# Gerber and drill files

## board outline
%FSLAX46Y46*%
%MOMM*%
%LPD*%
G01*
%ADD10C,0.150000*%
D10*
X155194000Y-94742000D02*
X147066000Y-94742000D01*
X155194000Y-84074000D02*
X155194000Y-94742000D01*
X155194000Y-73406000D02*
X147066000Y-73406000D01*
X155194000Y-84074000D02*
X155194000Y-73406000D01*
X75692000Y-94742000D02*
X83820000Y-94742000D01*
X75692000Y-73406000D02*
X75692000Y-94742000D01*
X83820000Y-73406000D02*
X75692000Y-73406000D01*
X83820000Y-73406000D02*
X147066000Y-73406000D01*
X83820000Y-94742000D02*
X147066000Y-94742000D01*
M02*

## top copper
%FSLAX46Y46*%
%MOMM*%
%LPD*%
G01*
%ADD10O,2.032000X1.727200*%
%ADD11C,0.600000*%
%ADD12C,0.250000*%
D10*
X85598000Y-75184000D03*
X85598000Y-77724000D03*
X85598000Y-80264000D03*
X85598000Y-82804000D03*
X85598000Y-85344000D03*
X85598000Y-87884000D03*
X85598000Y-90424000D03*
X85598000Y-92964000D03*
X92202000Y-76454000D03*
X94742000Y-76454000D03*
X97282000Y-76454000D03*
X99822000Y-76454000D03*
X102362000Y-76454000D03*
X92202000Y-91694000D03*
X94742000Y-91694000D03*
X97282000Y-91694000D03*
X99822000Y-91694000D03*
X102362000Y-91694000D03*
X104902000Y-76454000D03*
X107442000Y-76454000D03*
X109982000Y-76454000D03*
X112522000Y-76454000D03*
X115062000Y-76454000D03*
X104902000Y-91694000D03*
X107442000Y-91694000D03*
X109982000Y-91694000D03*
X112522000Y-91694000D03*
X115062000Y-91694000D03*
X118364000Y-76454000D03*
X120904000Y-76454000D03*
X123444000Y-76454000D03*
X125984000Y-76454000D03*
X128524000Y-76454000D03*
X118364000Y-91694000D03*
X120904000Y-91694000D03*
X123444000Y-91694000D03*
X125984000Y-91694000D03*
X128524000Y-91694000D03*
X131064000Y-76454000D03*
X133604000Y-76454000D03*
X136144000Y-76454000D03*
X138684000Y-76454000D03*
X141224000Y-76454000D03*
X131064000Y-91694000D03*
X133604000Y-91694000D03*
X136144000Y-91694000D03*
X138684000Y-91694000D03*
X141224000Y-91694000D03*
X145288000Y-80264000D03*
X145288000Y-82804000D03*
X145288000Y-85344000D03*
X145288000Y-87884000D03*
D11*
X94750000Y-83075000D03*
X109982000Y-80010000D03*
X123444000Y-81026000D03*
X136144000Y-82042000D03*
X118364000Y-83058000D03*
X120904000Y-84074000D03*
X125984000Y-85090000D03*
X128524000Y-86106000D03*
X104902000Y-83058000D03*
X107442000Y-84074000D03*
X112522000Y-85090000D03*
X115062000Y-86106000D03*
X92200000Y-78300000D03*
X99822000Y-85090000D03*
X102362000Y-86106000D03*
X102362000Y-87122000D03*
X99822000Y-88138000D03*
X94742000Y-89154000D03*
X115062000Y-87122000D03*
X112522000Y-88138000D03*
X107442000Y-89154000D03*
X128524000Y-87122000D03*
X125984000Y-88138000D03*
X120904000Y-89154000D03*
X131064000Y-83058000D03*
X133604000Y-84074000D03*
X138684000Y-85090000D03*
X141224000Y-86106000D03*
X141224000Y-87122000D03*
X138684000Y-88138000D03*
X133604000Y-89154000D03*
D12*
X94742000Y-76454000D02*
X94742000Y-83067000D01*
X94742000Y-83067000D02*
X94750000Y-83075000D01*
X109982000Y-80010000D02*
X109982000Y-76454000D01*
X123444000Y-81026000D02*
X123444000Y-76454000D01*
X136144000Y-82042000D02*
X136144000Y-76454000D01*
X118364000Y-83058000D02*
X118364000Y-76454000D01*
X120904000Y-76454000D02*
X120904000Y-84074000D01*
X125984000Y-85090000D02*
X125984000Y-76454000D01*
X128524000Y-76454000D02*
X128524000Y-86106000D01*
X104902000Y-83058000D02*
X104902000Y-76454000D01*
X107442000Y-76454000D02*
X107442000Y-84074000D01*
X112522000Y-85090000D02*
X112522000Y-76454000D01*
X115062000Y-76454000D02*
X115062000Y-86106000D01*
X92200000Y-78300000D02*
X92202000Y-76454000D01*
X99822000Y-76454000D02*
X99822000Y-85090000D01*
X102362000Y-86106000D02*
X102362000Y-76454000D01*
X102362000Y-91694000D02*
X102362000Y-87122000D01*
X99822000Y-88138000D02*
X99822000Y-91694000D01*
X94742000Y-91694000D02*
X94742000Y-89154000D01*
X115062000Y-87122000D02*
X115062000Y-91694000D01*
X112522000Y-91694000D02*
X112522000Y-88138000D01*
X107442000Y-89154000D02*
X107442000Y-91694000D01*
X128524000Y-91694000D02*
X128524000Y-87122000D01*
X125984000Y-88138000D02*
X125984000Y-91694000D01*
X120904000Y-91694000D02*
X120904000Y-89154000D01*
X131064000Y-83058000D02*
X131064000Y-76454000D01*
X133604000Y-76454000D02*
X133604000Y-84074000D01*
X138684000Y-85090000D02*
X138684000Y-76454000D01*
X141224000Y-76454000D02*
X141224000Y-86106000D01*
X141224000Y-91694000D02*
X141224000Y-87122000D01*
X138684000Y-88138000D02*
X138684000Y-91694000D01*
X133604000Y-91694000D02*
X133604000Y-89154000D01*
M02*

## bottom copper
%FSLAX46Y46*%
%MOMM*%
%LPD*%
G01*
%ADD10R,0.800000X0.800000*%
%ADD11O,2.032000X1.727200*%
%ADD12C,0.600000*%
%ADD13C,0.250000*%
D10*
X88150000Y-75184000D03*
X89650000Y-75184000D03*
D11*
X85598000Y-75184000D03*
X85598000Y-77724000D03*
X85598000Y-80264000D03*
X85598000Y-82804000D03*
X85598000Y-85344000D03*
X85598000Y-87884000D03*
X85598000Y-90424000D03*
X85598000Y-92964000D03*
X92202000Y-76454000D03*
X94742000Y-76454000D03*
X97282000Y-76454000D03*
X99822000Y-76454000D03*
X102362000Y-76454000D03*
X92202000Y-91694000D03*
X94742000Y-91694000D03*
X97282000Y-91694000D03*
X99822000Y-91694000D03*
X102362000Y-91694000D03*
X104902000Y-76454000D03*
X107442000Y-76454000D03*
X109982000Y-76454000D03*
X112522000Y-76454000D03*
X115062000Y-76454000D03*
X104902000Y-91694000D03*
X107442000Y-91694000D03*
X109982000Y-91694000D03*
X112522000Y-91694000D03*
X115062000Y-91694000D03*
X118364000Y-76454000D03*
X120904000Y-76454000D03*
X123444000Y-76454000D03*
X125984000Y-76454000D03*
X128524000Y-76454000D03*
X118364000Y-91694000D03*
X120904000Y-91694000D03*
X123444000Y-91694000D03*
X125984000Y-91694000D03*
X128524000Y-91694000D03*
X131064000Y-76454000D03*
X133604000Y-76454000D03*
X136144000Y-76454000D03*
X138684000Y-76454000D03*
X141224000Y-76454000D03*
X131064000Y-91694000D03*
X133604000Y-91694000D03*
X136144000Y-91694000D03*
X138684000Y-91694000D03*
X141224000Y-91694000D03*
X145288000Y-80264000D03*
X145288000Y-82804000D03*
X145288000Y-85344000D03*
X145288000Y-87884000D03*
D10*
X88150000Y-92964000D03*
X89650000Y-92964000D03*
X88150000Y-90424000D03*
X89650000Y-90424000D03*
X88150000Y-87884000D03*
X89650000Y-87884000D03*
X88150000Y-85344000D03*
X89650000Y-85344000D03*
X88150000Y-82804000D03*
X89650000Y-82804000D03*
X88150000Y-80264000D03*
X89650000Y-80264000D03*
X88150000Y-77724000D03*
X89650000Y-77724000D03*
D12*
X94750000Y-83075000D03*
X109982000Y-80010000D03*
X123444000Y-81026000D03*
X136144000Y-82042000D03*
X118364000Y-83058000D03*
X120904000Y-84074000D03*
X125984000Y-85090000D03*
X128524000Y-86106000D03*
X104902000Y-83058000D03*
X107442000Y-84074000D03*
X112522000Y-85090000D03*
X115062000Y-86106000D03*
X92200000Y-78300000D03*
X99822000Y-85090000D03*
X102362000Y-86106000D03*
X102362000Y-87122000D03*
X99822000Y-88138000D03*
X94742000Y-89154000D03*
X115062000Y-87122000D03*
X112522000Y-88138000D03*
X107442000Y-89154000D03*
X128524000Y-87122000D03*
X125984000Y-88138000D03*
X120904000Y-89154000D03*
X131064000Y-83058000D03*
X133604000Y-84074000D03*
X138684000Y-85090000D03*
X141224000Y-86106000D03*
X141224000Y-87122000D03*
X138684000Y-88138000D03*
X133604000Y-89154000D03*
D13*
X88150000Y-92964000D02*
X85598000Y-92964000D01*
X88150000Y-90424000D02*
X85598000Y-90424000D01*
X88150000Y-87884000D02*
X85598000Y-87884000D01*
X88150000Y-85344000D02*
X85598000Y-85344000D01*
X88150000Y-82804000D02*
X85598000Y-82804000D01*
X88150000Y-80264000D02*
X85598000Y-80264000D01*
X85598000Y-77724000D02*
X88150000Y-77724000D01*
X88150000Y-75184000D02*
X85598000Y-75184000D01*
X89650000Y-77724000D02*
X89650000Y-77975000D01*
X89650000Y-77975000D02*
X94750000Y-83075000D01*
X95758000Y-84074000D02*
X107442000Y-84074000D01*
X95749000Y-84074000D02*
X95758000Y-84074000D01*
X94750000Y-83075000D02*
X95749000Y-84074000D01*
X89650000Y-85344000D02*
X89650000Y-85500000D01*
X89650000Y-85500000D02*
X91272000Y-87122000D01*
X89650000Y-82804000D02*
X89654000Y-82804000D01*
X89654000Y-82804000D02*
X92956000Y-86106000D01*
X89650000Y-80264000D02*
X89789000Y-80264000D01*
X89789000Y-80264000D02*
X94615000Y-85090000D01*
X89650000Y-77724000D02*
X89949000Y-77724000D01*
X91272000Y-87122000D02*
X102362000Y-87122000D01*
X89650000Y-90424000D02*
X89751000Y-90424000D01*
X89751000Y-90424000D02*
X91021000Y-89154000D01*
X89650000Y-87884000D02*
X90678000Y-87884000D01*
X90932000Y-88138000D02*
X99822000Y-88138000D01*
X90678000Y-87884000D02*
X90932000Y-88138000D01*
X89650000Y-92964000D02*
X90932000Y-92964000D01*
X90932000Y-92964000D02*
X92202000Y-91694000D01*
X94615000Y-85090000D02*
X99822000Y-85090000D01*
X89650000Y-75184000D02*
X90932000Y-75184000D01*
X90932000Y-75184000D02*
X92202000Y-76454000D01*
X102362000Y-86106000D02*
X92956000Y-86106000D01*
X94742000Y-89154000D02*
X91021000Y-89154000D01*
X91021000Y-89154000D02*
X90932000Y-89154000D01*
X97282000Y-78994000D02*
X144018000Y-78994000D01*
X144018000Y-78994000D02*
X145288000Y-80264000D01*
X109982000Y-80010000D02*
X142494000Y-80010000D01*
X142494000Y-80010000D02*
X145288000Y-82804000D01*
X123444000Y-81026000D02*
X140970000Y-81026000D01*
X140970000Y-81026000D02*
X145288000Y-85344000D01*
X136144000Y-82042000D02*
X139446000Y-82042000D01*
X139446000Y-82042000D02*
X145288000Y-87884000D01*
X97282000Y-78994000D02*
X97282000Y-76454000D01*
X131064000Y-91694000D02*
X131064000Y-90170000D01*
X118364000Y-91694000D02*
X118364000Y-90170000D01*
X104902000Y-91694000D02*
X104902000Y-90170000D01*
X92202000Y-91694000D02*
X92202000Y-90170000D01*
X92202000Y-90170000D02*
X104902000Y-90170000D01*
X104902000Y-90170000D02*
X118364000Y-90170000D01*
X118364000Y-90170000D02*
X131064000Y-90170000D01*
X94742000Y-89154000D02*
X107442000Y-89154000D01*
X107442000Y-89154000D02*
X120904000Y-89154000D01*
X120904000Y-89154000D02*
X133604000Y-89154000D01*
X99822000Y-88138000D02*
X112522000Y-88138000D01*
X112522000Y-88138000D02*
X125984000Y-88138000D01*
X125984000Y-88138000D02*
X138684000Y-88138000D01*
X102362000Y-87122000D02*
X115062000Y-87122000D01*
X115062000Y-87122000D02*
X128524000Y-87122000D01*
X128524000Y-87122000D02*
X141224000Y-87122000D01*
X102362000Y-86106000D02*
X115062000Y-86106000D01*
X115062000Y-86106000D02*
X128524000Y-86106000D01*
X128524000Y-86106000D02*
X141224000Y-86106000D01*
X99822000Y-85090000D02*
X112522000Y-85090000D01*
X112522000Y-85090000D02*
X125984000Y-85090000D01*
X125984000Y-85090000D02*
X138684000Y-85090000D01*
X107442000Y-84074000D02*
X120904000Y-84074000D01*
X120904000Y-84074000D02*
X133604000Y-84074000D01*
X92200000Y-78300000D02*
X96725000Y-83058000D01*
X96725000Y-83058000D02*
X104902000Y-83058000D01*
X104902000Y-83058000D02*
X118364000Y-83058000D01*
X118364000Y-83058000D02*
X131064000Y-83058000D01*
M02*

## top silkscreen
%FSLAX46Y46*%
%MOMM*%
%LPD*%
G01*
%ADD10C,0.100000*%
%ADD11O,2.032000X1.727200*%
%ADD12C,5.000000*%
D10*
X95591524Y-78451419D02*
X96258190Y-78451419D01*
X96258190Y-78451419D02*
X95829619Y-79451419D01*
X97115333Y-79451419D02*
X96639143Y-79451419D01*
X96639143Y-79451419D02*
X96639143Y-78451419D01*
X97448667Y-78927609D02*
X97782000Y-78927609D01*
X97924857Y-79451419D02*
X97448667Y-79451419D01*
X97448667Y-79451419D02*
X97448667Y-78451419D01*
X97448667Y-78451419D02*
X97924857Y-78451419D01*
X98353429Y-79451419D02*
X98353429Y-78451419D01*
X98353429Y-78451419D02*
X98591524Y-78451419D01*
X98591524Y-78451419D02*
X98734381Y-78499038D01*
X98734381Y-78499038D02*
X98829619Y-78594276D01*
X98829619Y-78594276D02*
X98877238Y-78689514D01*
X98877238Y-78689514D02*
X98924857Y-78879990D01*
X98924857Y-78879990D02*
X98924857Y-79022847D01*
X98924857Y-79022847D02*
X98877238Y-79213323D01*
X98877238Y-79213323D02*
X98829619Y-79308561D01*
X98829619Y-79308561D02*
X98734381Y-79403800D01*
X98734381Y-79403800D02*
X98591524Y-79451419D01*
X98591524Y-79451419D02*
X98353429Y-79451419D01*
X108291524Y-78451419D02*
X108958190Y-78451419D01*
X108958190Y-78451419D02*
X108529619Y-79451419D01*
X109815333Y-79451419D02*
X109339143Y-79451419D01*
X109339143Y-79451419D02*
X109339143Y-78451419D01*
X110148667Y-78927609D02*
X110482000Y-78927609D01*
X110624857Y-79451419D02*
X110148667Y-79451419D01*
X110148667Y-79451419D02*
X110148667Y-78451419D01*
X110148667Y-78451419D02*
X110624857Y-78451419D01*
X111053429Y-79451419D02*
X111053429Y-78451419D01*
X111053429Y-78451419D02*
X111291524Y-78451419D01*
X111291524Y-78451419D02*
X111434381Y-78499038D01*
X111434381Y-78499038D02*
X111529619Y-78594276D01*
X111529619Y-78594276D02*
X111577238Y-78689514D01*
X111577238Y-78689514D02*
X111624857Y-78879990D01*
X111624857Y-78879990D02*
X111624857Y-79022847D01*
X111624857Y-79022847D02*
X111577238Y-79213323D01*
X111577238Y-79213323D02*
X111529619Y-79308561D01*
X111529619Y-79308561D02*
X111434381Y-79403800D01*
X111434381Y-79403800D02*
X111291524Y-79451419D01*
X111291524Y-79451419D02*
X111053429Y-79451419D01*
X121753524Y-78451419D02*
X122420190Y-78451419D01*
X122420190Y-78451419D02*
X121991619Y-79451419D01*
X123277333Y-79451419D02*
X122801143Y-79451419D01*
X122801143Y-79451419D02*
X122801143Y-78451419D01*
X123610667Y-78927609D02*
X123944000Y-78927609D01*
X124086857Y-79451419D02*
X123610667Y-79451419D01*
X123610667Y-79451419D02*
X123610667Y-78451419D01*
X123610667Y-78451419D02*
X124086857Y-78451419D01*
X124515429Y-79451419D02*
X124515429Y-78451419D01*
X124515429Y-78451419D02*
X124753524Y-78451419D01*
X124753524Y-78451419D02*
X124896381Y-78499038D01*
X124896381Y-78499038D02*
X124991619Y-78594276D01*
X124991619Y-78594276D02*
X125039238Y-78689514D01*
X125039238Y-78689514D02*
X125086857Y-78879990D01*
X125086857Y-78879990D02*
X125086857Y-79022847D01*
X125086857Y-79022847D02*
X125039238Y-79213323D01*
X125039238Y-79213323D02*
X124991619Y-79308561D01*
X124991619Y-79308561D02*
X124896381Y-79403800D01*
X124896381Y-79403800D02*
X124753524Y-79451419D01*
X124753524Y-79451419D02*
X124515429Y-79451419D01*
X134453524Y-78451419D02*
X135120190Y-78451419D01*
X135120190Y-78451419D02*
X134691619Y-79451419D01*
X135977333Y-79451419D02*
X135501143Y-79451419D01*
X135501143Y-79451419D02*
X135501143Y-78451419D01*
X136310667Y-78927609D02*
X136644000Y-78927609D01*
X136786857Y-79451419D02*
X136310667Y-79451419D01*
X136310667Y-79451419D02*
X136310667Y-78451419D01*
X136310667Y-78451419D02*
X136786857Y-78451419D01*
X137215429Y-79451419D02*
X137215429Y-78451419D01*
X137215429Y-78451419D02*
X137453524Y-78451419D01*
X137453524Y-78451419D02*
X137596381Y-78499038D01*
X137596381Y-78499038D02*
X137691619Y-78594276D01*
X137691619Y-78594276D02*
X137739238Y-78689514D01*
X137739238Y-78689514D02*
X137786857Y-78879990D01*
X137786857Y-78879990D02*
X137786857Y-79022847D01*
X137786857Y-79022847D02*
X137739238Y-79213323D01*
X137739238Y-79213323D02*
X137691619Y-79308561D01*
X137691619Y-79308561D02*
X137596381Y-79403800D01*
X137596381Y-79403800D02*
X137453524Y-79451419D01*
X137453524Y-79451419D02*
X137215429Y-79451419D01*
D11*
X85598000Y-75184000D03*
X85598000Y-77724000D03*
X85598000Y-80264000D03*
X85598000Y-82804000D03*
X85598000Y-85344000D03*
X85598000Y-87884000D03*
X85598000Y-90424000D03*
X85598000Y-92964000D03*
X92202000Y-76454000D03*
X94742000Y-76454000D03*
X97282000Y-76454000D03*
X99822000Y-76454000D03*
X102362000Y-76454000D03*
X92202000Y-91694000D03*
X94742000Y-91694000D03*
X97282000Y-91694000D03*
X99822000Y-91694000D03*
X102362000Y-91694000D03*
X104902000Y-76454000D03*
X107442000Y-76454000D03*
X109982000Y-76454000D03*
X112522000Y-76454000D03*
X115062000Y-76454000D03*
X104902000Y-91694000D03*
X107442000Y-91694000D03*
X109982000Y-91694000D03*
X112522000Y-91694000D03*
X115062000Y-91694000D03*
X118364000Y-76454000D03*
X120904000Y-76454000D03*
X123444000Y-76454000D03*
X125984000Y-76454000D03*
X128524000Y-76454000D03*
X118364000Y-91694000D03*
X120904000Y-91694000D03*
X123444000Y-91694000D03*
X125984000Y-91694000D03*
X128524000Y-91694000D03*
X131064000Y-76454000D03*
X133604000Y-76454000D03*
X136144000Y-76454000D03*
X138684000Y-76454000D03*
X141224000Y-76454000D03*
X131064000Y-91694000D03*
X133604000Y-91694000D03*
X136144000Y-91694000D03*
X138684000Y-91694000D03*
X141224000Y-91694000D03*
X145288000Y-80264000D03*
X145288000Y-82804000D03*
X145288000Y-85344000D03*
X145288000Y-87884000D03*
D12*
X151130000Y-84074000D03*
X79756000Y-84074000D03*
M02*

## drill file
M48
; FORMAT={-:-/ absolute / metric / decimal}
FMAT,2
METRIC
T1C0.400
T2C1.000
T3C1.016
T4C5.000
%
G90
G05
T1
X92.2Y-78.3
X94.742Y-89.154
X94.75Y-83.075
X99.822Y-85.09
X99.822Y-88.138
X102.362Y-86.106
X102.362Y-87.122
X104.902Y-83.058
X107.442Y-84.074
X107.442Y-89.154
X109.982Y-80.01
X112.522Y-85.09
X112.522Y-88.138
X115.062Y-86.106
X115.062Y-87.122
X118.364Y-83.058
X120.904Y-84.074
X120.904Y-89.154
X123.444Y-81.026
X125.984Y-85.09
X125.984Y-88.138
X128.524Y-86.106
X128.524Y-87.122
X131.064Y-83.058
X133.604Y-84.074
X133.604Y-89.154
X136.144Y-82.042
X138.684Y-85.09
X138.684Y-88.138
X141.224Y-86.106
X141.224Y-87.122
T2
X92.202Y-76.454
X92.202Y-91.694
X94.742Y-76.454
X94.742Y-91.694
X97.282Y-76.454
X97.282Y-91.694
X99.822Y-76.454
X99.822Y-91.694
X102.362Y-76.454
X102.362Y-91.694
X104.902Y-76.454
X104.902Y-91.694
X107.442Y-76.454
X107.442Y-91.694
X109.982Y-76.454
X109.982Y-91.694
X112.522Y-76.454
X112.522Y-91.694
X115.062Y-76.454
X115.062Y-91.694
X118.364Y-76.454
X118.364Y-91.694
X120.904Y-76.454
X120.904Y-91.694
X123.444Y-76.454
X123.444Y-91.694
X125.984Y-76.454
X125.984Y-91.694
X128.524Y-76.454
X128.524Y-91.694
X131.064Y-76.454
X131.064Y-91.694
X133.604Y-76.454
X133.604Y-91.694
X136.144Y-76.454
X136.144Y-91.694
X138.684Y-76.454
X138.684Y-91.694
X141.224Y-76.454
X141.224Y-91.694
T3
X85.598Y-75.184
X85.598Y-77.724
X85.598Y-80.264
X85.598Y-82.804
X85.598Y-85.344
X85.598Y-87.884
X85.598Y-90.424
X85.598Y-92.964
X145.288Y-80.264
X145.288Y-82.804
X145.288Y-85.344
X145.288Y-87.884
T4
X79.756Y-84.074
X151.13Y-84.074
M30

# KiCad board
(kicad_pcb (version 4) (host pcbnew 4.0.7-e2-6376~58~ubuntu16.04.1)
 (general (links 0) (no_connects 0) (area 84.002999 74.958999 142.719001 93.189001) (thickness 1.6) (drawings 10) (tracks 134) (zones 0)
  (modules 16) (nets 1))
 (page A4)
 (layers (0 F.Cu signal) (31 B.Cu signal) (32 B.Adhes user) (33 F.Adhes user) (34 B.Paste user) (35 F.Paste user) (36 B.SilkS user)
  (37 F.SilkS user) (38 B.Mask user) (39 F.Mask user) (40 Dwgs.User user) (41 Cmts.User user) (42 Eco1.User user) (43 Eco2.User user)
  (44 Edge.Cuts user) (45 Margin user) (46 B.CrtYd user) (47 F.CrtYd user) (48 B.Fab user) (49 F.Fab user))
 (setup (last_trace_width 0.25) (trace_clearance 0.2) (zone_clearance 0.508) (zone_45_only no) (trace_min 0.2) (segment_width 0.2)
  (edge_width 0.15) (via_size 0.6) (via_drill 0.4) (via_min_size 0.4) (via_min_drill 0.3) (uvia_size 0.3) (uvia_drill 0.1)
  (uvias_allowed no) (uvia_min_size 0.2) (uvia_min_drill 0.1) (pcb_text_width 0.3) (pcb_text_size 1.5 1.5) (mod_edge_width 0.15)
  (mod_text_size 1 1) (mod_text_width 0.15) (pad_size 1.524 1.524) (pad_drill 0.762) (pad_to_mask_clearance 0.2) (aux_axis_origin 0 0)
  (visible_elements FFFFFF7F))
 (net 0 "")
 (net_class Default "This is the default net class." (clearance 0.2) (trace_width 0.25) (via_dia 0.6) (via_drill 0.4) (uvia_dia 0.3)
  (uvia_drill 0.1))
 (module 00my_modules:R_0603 (layer B.Cu) (at 88.9 75.184)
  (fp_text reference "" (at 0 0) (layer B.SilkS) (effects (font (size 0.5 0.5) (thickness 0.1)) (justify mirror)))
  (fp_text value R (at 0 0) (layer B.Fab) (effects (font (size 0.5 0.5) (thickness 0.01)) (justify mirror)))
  (pad 1 smd rect (at -0.75 0) (size 0.8 0.8) (layers B.Cu B.Paste B.Mask))
  (pad 2 smd rect (at 0.75 0) (size 0.8 0.8) (layers B.Cu B.Paste B.Mask)))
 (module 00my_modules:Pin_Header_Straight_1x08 (layer F.Cu) (at 85.598 75.184)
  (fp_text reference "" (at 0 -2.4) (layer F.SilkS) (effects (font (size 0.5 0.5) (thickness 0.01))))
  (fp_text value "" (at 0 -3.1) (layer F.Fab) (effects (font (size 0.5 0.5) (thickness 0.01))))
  (pad 1 thru_hole oval (at 0 0) (size 2.032 1.7272) (drill 1.016) (layers *.Cu *.Mask F.SilkS))
  (pad 2 thru_hole oval (at 0 2.54) (size 2.032 1.7272) (drill 1.016) (layers *.Cu *.Mask F.SilkS))
  (pad 3 thru_hole oval (at 0 5.08) (size 2.032 1.7272) (drill 1.016) (layers *.Cu *.Mask F.SilkS))
  (pad 4 thru_hole oval (at 0 7.62) (size 2.032 1.7272) (drill 1.016) (layers *.Cu *.Mask F.SilkS))
  (pad 5 thru_hole oval (at 0 10.16) (size 2.032 1.7272) (drill 1.016) (layers *.Cu *.Mask F.SilkS))
  (pad 6 thru_hole oval (at 0 12.7) (size 2.032 1.7272) (drill 1.016) (layers *.Cu *.Mask F.SilkS))
  (pad 7 thru_hole oval (at 0 15.24) (size 2.032 1.7272) (drill 1.016) (layers *.Cu *.Mask F.SilkS))
  (pad 8 thru_hole oval (at 0 17.78) (size 2.032 1.7272) (drill 1.016) (layers *.Cu *.Mask F.SilkS)))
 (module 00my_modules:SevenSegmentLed (layer F.Cu) (at 92.202 76.454)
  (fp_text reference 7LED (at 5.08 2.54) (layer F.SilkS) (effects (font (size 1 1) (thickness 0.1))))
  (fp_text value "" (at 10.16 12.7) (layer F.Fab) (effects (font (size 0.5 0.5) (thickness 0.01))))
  (pad 10 thru_hole oval (at 0 0) (size 2.032 1.7272) (drill 1) (layers *.Cu *.Mask F.SilkS))
  (pad 9 thru_hole oval (at 2.54 0) (size 2.032 1.7272) (drill 1) (layers *.Cu *.Mask F.SilkS))
  (pad 8 thru_hole oval (at 5.08 0) (size 2.032 1.7272) (drill 1) (layers *.Cu *.Mask F.SilkS))
  (pad 7 thru_hole oval (at 7.62 0) (size 2.032 1.7272) (drill 1) (layers *.Cu *.Mask F.SilkS))
  (pad 6 thru_hole oval (at 10.16 0) (size 2.032 1.7272) (drill 1) (layers *.Cu *.Mask F.SilkS))
  (pad 1 thru_hole oval (at 0 15.24) (size 2.032 1.7272) (drill 1) (layers *.Cu *.Mask F.SilkS))
  (pad 2 thru_hole oval (at 2.54 15.24) (size 2.032 1.7272) (drill 1) (layers *.Cu *.Mask F.SilkS))
  (pad 3 thru_hole oval (at 5.08 15.24) (size 2.032 1.7272) (drill 1) (layers *.Cu *.Mask F.SilkS))
  (pad 4 thru_hole oval (at 7.62 15.24) (size 2.032 1.7272) (drill 1) (layers *.Cu *.Mask F.SilkS))
  (pad 5 thru_hole oval (at 10.16 15.24) (size 2.032 1.7272) (drill 1) (layers *.Cu *.Mask F.SilkS)))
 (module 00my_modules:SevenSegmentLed (layer F.Cu) (at 104.902 76.454)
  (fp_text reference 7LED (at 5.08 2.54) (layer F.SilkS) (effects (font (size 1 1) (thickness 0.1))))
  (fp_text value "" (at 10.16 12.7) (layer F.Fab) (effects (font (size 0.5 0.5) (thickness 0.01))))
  (pad 10 thru_hole oval (at 0 0) (size 2.032 1.7272) (drill 1) (layers *.Cu *.Mask F.SilkS))
  (pad 9 thru_hole oval (at 2.54 0) (size 2.032 1.7272) (drill 1) (layers *.Cu *.Mask F.SilkS))
  (pad 8 thru_hole oval (at 5.08 0) (size 2.032 1.7272) (drill 1) (layers *.Cu *.Mask F.SilkS))
  (pad 7 thru_hole oval (at 7.62 0) (size 2.032 1.7272) (drill 1) (layers *.Cu *.Mask F.SilkS))
  (pad 6 thru_hole oval (at 10.16 0) (size 2.032 1.7272) (drill 1) (layers *.Cu *.Mask F.SilkS))
  (pad 1 thru_hole oval (at 0 15.24) (size 2.032 1.7272) (drill 1) (layers *.Cu *.Mask F.SilkS))
  (pad 2 thru_hole oval (at 2.54 15.24) (size 2.032 1.7272) (drill 1) (layers *.Cu *.Mask F.SilkS))
  (pad 3 thru_hole oval (at 5.08 15.24) (size 2.032 1.7272) (drill 1) (layers *.Cu *.Mask F.SilkS))
  (pad 4 thru_hole oval (at 7.62 15.24) (size 2.032 1.7272) (drill 1) (layers *.Cu *.Mask F.SilkS))
  (pad 5 thru_hole oval (at 10.16 15.24) (size 2.032 1.7272) (drill 1) (layers *.Cu *.Mask F.SilkS)))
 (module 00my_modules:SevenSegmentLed (layer F.Cu) (at 118.364 76.454)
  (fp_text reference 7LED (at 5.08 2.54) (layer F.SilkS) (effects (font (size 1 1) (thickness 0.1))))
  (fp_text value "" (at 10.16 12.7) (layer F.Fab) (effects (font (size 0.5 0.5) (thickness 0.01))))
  (pad 10 thru_hole oval (at 0 0) (size 2.032 1.7272) (drill 1) (layers *.Cu *.Mask F.SilkS))
  (pad 9 thru_hole oval (at 2.54 0) (size 2.032 1.7272) (drill 1) (layers *.Cu *.Mask F.SilkS))
  (pad 8 thru_hole oval (at 5.08 0) (size 2.032 1.7272) (drill 1) (layers *.Cu *.Mask F.SilkS))
  (pad 7 thru_hole oval (at 7.62 0) (size 2.032 1.7272) (drill 1) (layers *.Cu *.Mask F.SilkS))
  (pad 6 thru_hole oval (at 10.16 0) (size 2.032 1.7272) (drill 1) (layers *.Cu *.Mask F.SilkS))
  (pad 1 thru_hole oval (at 0 15.24) (size 2.032 1.7272) (drill 1) (layers *.Cu *.Mask F.SilkS))
  (pad 2 thru_hole oval (at 2.54 15.24) (size 2.032 1.7272) (drill 1) (layers *.Cu *.Mask F.SilkS))
  (pad 3 thru_hole oval (at 5.08 15.24) (size 2.032 1.7272) (drill 1) (layers *.Cu *.Mask F.SilkS))
  (pad 4 thru_hole oval (at 7.62 15.24) (size 2.032 1.7272) (drill 1) (layers *.Cu *.Mask F.SilkS))
  (pad 5 thru_hole oval (at 10.16 15.24) (size 2.032 1.7272) (drill 1) (layers *.Cu *.Mask F.SilkS)))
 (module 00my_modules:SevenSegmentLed (layer F.Cu) (at 131.064 76.454)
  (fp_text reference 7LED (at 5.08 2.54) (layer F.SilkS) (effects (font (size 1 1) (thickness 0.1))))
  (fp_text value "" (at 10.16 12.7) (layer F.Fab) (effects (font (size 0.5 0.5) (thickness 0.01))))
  (pad 10 thru_hole oval (at 0 0) (size 2.032 1.7272) (drill 1) (layers *.Cu *.Mask F.SilkS))
  (pad 9 thru_hole oval (at 2.54 0) (size 2.032 1.7272) (drill 1) (layers *.Cu *.Mask F.SilkS))
  (pad 8 thru_hole oval (at 5.08 0) (size 2.032 1.7272) (drill 1) (layers *.Cu *.Mask F.SilkS))
  (pad 7 thru_hole oval (at 7.62 0) (size 2.032 1.7272) (drill 1) (layers *.Cu *.Mask F.SilkS))
  (pad 6 thru_hole oval (at 10.16 0) (size 2.032 1.7272) (drill 1) (layers *.Cu *.Mask F.SilkS))
  (pad 1 thru_hole oval (at 0 15.24) (size 2.032 1.7272) (drill 1) (layers *.Cu *.Mask F.SilkS))
  (pad 2 thru_hole oval (at 2.54 15.24) (size 2.032 1.7272) (drill 1) (layers *.Cu *.Mask F.SilkS))
  (pad 3 thru_hole oval (at 5.08 15.24) (size 2.032 1.7272) (drill 1) (layers *.Cu *.Mask F.SilkS))
  (pad 4 thru_hole oval (at 7.62 15.24) (size 2.032 1.7272) (drill 1) (layers *.Cu *.Mask F.SilkS))
  (pad 5 thru_hole oval (at 10.16 15.24) (size 2.032 1.7272) (drill 1) (layers *.Cu *.Mask F.SilkS)))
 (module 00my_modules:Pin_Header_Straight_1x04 (layer F.Cu) (at 145.288 80.264)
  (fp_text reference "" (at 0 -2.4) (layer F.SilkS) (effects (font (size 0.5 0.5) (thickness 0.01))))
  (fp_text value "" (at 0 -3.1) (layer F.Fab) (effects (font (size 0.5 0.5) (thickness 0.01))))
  (pad 1 thru_hole oval (at 0 0) (size 2.032 1.7272) (drill 1.016) (layers *.Cu *.Mask F.SilkS))
  (pad 2 thru_hole oval (at 0 2.54) (size 2.032 1.7272) (drill 1.016) (layers *.Cu *.Mask F.SilkS))
  (pad 3 thru_hole oval (at 0 5.08) (size 2.032 1.7272) (drill 1.016) (layers *.Cu *.Mask F.SilkS))
  (pad 4 thru_hole oval (at 0 7.62) (size 2.032 1.7272) (drill 1.016) (layers *.Cu *.Mask F.SilkS)))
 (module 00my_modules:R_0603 (layer B.Cu) (at 88.9 92.964)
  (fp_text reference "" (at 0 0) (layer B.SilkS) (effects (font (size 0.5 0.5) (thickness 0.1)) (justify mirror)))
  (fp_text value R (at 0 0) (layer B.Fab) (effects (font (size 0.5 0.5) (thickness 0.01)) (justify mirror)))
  (pad 1 smd rect (at -0.75 0) (size 0.8 0.8) (layers B.Cu B.Paste B.Mask))
  (pad 2 smd rect (at 0.75 0) (size 0.8 0.8) (layers B.Cu B.Paste B.Mask)))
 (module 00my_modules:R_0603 (layer B.Cu) (at 88.9 90.424)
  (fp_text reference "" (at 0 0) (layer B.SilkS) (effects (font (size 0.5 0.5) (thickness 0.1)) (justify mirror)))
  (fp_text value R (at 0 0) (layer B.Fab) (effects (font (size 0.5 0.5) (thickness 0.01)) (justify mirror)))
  (pad 1 smd rect (at -0.75 0) (size 0.8 0.8) (layers B.Cu B.Paste B.Mask))
  (pad 2 smd rect (at 0.75 0) (size 0.8 0.8) (layers B.Cu B.Paste B.Mask)))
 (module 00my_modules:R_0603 (layer B.Cu) (at 88.9 87.884)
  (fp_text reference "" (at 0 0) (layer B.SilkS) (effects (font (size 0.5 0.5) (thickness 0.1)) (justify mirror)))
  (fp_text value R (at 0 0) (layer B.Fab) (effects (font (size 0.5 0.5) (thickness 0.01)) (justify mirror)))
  (pad 1 smd rect (at -0.75 0) (size 0.8 0.8) (layers B.Cu B.Paste B.Mask))
  (pad 2 smd rect (at 0.75 0) (size 0.8 0.8) (layers B.Cu B.Paste B.Mask)))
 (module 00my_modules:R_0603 (layer B.Cu) (at 88.9 85.344)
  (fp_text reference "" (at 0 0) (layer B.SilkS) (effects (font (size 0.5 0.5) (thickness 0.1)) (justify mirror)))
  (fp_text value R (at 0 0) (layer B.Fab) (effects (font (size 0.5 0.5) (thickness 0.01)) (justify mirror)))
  (pad 1 smd rect (at -0.75 0) (size 0.8 0.8) (layers B.Cu B.Paste B.Mask))
  (pad 2 smd rect (at 0.75 0) (size 0.8 0.8) (layers B.Cu B.Paste B.Mask)))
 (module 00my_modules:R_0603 (layer B.Cu) (at 88.9 82.804)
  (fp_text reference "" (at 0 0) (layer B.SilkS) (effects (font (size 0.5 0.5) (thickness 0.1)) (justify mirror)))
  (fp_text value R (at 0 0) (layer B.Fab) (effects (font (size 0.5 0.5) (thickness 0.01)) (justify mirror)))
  (pad 1 smd rect (at -0.75 0) (size 0.8 0.8) (layers B.Cu B.Paste B.Mask))
  (pad 2 smd rect (at 0.75 0) (size 0.8 0.8) (layers B.Cu B.Paste B.Mask)))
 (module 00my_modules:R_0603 (layer B.Cu) (at 88.9 80.264)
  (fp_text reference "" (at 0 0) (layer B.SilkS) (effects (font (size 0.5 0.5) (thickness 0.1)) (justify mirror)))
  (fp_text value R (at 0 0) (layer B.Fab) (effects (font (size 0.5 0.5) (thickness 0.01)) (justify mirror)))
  (pad 1 smd rect (at -0.75 0) (size 0.8 0.8) (layers B.Cu B.Paste B.Mask))
  (pad 2 smd rect (at 0.75 0) (size 0.8 0.8) (layers B.Cu B.Paste B.Mask)))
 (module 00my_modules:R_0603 (layer B.Cu) (at 88.9 77.724)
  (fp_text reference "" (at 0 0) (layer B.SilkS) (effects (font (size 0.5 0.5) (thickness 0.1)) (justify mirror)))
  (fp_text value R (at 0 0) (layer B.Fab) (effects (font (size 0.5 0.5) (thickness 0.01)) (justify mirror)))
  (pad 1 smd rect (at -0.75 0) (size 0.8 0.8) (layers B.Cu B.Paste B.Mask))
  (pad 2 smd rect (at 0.75 0) (size 0.8 0.8) (layers B.Cu B.Paste B.Mask)))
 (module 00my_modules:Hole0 (layer F.Cu) (at 151.13 84.074)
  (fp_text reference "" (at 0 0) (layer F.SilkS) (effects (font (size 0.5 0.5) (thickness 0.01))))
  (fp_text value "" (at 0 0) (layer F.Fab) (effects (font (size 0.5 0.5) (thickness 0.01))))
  (pad "" np_thru_hole circle (at 0 0) (size 5 5) (drill 5) (layers *.Cu *.Mask F.SilkS)))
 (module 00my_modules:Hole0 (layer F.Cu) (at 79.756 84.074)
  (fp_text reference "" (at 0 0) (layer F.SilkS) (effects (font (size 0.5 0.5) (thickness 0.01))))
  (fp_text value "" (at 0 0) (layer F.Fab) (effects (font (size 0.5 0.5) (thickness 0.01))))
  (pad "" np_thru_hole circle (at 0 0) (size 5 5) (drill 5) (layers *.Cu *.Mask F.SilkS)))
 (gr_line (start 155.194 94.742) (end 147.066 94.742) (angle 90) (layer Edge.Cuts) (width 0.15))
 (gr_line (start 155.194 84.074) (end 155.194 94.742) (angle 90) (layer Edge.Cuts) (width 0.15))
 (gr_line (start 155.194 73.406) (end 147.066 73.406) (angle 90) (layer Edge.Cuts) (width 0.15))
 (gr_line (start 155.194 84.074) (end 155.194 73.406) (angle 90) (layer Edge.Cuts) (width 0.15))
 (gr_line (start 75.692 94.742) (end 83.82 94.742) (angle 90) (layer Edge.Cuts) (width 0.15))
 (gr_line (start 75.692 73.406) (end 75.692 94.742) (angle 90) (layer Edge.Cuts) (width 0.15))
 (gr_line (start 83.82 73.406) (end 75.692 73.406) (angle 90) (layer Edge.Cuts) (width 0.15))
 (gr_line (start 83.82 73.406) (end 147.066 73.406) (angle 90) (layer Edge.Cuts) (width 0.15))
 (gr_line (start 83.82 94.742) (end 147.066 94.742) (angle 90) (layer Edge.Cuts) (width 0.15))
 (segment (start 88.15 92.964) (end 85.598 92.964) (width 0.25) (layer B.Cu) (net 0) (status C00000))
 (segment (start 88.15 90.424) (end 85.598 90.424) (width 0.25) (layer B.Cu) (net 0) (status C00000))
 (segment (start 88.15 87.884) (end 85.598 87.884) (width 0.25) (layer B.Cu) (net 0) (status C00000))
 (segment (start 88.15 85.344) (end 85.598 85.344) (width 0.25) (layer B.Cu) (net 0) (status C00000))
 (segment (start 88.15 82.804) (end 85.598 82.804) (width 0.25) (layer B.Cu) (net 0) (status C00000))
 (segment (start 88.15 80.264) (end 85.598 80.264) (width 0.25) (layer B.Cu) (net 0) (status C00000))
 (segment (start 85.598 77.724) (end 88.15 77.724) (width 0.25) (layer B.Cu) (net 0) (status C00000))
 (segment (start 88.15 75.184) (end 85.598 75.184) (width 0.25) (layer B.Cu) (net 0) (status C00000))
 (segment (start 89.65 77.724) (end 89.65 77.975) (width 0.25) (layer B.Cu) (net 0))
 (segment (start 89.65 77.975) (end 94.75 83.075) (width 0.25) (layer B.Cu) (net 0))
 (segment (start 94.742 76.454) (end 94.742 83.067) (width 0.25) (layer F.Cu) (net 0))
 (segment (start 95.758 84.074) (end 107.442 84.074) (width 0.25) (layer B.Cu) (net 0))
 (segment (start 95.749 84.074) (end 95.758 84.074) (width 0.25) (layer B.Cu) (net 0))
 (segment (start 94.75 83.075) (end 95.749 84.074) (width 0.25) (layer B.Cu) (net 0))
 (via (at 94.75 83.075) (size 0.6) (drill 0.4) (layers F.Cu B.Cu) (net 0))
 (segment (start 94.742 83.067) (end 94.75 83.075) (width 0.25) (layer F.Cu) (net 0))
 (segment (start 89.65 85.344) (end 89.65 85.5) (width 0.25) (layer B.Cu) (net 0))
 (segment (start 89.65 85.5) (end 91.272 87.122) (width 0.25) (layer B.Cu) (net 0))
 (segment (start 89.65 82.804) (end 89.654 82.804) (width 0.25) (layer B.Cu) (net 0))
 (segment (start 89.654 82.804) (end 92.956 86.106) (width 0.25) (layer B.Cu) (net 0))
 (segment (start 89.65 80.264) (end 89.789 80.264) (width 0.25) (layer B.Cu) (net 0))
 (segment (start 89.789 80.264) (end 94.615 85.09) (width 0.25) (layer B.Cu) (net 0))
 (segment (start 89.65 77.724) (end 89.949 77.724) (width 0.25) (layer B.Cu) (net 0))
 (segment (start 91.272 87.122) (end 102.362 87.122) (width 0.25) (layer B.Cu) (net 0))
 (segment (start 89.65 90.424) (end 89.751 90.424) (width 0.25) (layer B.Cu) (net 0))
 (segment (start 89.751 90.424) (end 91.021 89.154) (width 0.25) (layer B.Cu) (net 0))
 (segment (start 89.65 87.884) (end 90.678 87.884) (width 0.25) (layer B.Cu) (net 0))
 (segment (start 90.932 88.138) (end 99.822 88.138) (width 0.25) (layer B.Cu) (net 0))
 (segment (start 90.678 87.884) (end 90.932 88.138) (width 0.25) (layer B.Cu) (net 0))
 (segment (start 89.65 92.964) (end 90.932 92.964) (width 0.25) (layer B.Cu) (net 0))
 (segment (start 90.932 92.964) (end 92.202 91.694) (width 0.25) (layer B.Cu) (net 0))
 (segment (start 94.615 85.09) (end 99.822 85.09) (width 0.25) (layer B.Cu) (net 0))
 (segment (start 89.65 75.184) (end 90.932 75.184) (width 0.25) (layer B.Cu) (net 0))
 (segment (start 90.932 75.184) (end 92.202 76.454) (width 0.25) (layer B.Cu) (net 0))
 (segment (start 102.362 86.106) (end 92.956 86.106) (width 0.25) (layer B.Cu) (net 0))
 (segment (start 94.742 89.154) (end 91.021 89.154) (width 0.25) (layer B.Cu) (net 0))
 (segment (start 91.021 89.154) (end 90.932 89.154) (width 0.25) (layer B.Cu) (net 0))
 (segment (start 97.282 78.994) (end 144.018 78.994) (width 0.25) (layer B.Cu) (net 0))
 (segment (start 144.018 78.994) (end 145.288 80.264) (width 0.25) (layer B.Cu) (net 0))
 (segment (start 109.982 80.01) (end 142.494 80.01) (width 0.25) (layer B.Cu) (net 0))
 (segment (start 142.494 80.01) (end 145.288 82.804) (width 0.25) (layer B.Cu) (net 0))
 (segment (start 123.444 81.026) (end 140.97 81.026) (width 0.25) (layer B.Cu) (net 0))
 (segment (start 140.97 81.026) (end 145.288 85.344) (width 0.25) (layer B.Cu) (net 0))
 (segment (start 136.144 82.042) (end 139.446 82.042) (width 0.25) (layer B.Cu) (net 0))
 (segment (start 139.446 82.042) (end 145.288 87.884) (width 0.25) (layer B.Cu) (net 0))
 (segment (start 97.282 78.994) (end 97.282 76.454) (width 0.25) (layer B.Cu) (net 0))
 (via (at 109.982 80.01) (size 0.6) (drill 0.4) (layers F.Cu B.Cu) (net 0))
 (segment (start 109.982 80.01) (end 109.982 76.454) (width 0.25) (layer F.Cu) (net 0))
 (segment (start 123.444 81.026) (end 123.444 76.454) (width 0.25) (layer F.Cu) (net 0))
 (via (at 123.444 81.026) (size 0.6) (drill 0.4) (layers F.Cu B.Cu) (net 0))
 (via (at 136.144 82.042) (size 0.6) (drill 0.4) (layers F.Cu B.Cu) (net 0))
 (segment (start 136.144 82.042) (end 136.144 76.454) (width 0.25) (layer F.Cu) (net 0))
 (via (at 118.364 83.058) (size 0.6) (drill 0.4) (layers F.Cu B.Cu) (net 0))
 (segment (start 118.364 83.058) (end 118.364 76.454) (width 0.25) (layer F.Cu) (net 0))
 (segment (start 120.904 76.454) (end 120.904 84.074) (width 0.25) (layer F.Cu) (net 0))
 (via (at 120.904 84.074) (size 0.6) (drill 0.4) (layers F.Cu B.Cu) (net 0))
 (via (at 125.984 85.09) (size 0.6) (drill 0.4) (layers F.Cu B.Cu) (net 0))
 (segment (start 125.984 85.09) (end 125.984 76.454) (width 0.25) (layer F.Cu) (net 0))
 (segment (start 128.524 76.454) (end 128.524 86.106) (width 0.25) (layer F.Cu) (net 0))
 (via (at 128.524 86.106) (size 0.6) (drill 0.4) (layers F.Cu B.Cu) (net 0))
 (via (at 104.902 83.058) (size 0.6) (drill 0.4) (layers F.Cu B.Cu) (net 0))
 (segment (start 104.902 83.058) (end 104.902 76.454) (width 0.25) (layer F.Cu) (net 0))
 (segment (start 107.442 76.454) (end 107.442 84.074) (width 0.25) (layer F.Cu) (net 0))
 (via (at 107.442 84.074) (size 0.6) (drill 0.4) (layers F.Cu B.Cu) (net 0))
 (via (at 112.522 85.09) (size 0.6) (drill 0.4) (layers F.Cu B.Cu) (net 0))
 (segment (start 112.522 85.09) (end 112.522 76.454) (width 0.25) (layer F.Cu) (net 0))
 (segment (start 115.062 76.454) (end 115.062 86.106) (width 0.25) (layer F.Cu) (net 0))
 (via (at 115.062 86.106) (size 0.6) (drill 0.4) (layers F.Cu B.Cu) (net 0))
 (via (at 92.2 78.3) (size 0.6) (drill 0.4) (layers F.Cu B.Cu) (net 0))
 (segment (start 92.2 78.3) (end 92.202 76.454) (width 0.25) (layer F.Cu) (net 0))
 (segment (start 99.822 76.454) (end 99.822 85.09) (width 0.25) (layer F.Cu) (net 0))
 (via (at 99.822 85.09) (size 0.6) (drill 0.4) (layers F.Cu B.Cu) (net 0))
 (via (at 102.362 86.106) (size 0.6) (drill 0.4) (layers F.Cu B.Cu) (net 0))
 (segment (start 102.362 86.106) (end 102.362 76.454) (width 0.25) (layer F.Cu) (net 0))
 (segment (start 102.362 91.694) (end 102.362 87.122) (width 0.25) (layer F.Cu) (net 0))
 (via (at 102.362 87.122) (size 0.6) (drill 0.4) (layers F.Cu B.Cu) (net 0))
 (via (at 99.822 88.138) (size 0.6) (drill 0.4) (layers F.Cu B.Cu) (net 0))
 (segment (start 99.822 88.138) (end 99.822 91.694) (width 0.25) (layer F.Cu) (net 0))
 (segment (start 94.742 91.694) (end 94.742 89.154) (width 0.25) (layer F.Cu) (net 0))
 (via (at 94.742 89.154) (size 0.6) (drill 0.4) (layers F.Cu B.Cu) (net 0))
 (via (at 115.062 87.122) (size 0.6) (drill 0.4) (layers F.Cu B.Cu) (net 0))
 (segment (start 115.062 87.122) (end 115.062 91.694) (width 0.25) (layer F.Cu) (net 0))
 (segment (start 112.522 91.694) (end 112.522 88.138) (width 0.25) (layer F.Cu) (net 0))
 (via (at 112.522 88.138) (size 0.6) (drill 0.4) (layers F.Cu B.Cu) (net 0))
 (via (at 107.442 89.154) (size 0.6) (drill 0.4) (layers F.Cu B.Cu) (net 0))
 (segment (start 107.442 89.154) (end 107.442 91.694) (width 0.25) (layer F.Cu) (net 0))
 (segment (start 128.524 91.694) (end 128.524 87.122) (width 0.25) (layer F.Cu) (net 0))
 (via (at 128.524 87.122) (size 0.6) (drill 0.4) (layers F.Cu B.Cu) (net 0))
 (via (at 125.984 88.138) (size 0.6) (drill 0.4) (layers F.Cu B.Cu) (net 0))
 (segment (start 125.984 88.138) (end 125.984 91.694) (width 0.25) (layer F.Cu) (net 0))
 (segment (start 120.904 91.694) (end 120.904 89.154) (width 0.25) (layer F.Cu) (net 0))
 (via (at 120.904 89.154) (size 0.6) (drill 0.4) (layers F.Cu B.Cu) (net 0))
 (via (at 131.064 83.058) (size 0.6) (drill 0.4) (layers F.Cu B.Cu) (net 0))
 (segment (start 131.064 83.058) (end 131.064 76.454) (width 0.25) (layer F.Cu) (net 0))
 (segment (start 133.604 76.454) (end 133.604 84.074) (width 0.25) (layer F.Cu) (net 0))
 (via (at 133.604 84.074) (size 0.6) (drill 0.4) (layers F.Cu B.Cu) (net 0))
 (via (at 138.684 85.09) (size 0.6) (drill 0.4) (layers F.Cu B.Cu) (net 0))
 (segment (start 138.684 85.09) (end 138.684 76.454) (width 0.25) (layer F.Cu) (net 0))
 (segment (start 141.224 76.454) (end 141.224 86.106) (width 0.25) (layer F.Cu) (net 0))
 (via (at 141.224 86.106) (size 0.6) (drill 0.4) (layers F.Cu B.Cu) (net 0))
 (segment (start 141.224 91.694) (end 141.224 87.122) (width 0.25) (layer F.Cu) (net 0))
 (via (at 141.224 87.122) (size 0.6) (drill 0.4) (layers F.Cu B.Cu) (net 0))
 (via (at 138.684 88.138) (size 0.6) (drill 0.4) (layers F.Cu B.Cu) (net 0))
 (segment (start 138.684 88.138) (end 138.684 91.694) (width 0.25) (layer F.Cu) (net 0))
 (segment (start 133.604 91.694) (end 133.604 89.154) (width 0.25) (layer F.Cu) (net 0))
 (via (at 133.604 89.154) (size 0.6) (drill 0.4) (layers F.Cu B.Cu) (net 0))
 (segment (start 131.064 91.694) (end 131.064 90.17) (width 0.25) (layer B.Cu) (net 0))
 (segment (start 118.364 91.694) (end 118.364 90.17) (width 0.25) (layer B.Cu) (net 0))
 (segment (start 104.902 91.694) (end 104.902 90.17) (width 0.25) (layer B.Cu) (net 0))
 (segment (start 92.202 91.694) (end 92.202 90.17) (width 0.25) (layer B.Cu) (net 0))
 (segment (start 92.202 90.17) (end 104.902 90.17) (width 0.25) (layer B.Cu) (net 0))
 (segment (start 104.902 90.17) (end 118.364 90.17) (width 0.25) (layer B.Cu) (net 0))
 (segment (start 118.364 90.17) (end 131.064 90.17) (width 0.25) (layer B.Cu) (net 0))
 (segment (start 94.742 89.154) (end 107.442 89.154) (width 0.25) (layer B.Cu) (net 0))
 (segment (start 107.442 89.154) (end 120.904 89.154) (width 0.25) (layer B.Cu) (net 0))
 (segment (start 120.904 89.154) (end 133.604 89.154) (width 0.25) (layer B.Cu) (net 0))
 (segment (start 99.822 88.138) (end 112.522 88.138) (width 0.25) (layer B.Cu) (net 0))
 (segment (start 112.522 88.138) (end 125.984 88.138) (width 0.25) (layer B.Cu) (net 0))
 (segment (start 125.984 88.138) (end 138.684 88.138) (width 0.25) (layer B.Cu) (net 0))
 (segment (start 102.362 87.122) (end 115.062 87.122) (width 0.25) (layer B.Cu) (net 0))
 (segment (start 115.062 87.122) (end 128.524 87.122) (width 0.25) (layer B.Cu) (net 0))
 (segment (start 128.524 87.122) (end 141.224 87.122) (width 0.25) (layer B.Cu) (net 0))
 (segment (start 102.362 86.106) (end 115.062 86.106) (width 0.25) (layer B.Cu) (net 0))
 (segment (start 115.062 86.106) (end 128.524 86.106) (width 0.25) (layer B.Cu) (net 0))
 (segment (start 128.524 86.106) (end 141.224 86.106) (width 0.25) (layer B.Cu) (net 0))
 (segment (start 99.822 85.09) (end 112.522 85.09) (width 0.25) (layer B.Cu) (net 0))
 (segment (start 112.522 85.09) (end 125.984 85.09) (width 0.25) (layer B.Cu) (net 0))
 (segment (start 125.984 85.09) (end 138.684 85.09) (width 0.25) (layer B.Cu) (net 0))
 (segment (start 107.442 84.074) (end 120.904 84.074) (width 0.25) (layer B.Cu) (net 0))
 (segment (start 120.904 84.074) (end 133.604 84.074) (width 0.25) (layer B.Cu) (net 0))
 (segment (start 92.2 78.3) (end 96.725 83.058) (width 0.25) (layer B.Cu) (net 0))
 (segment (start 96.725 83.058) (end 104.902 83.058) (width 0.25) (layer B.Cu) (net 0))
 (segment (start 104.902 83.058) (end 118.364 83.058) (width 0.25) (layer B.Cu) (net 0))
 (segment (start 118.364 83.058) (end 131.064 83.058) (width 0.25) (layer B.Cu) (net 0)))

